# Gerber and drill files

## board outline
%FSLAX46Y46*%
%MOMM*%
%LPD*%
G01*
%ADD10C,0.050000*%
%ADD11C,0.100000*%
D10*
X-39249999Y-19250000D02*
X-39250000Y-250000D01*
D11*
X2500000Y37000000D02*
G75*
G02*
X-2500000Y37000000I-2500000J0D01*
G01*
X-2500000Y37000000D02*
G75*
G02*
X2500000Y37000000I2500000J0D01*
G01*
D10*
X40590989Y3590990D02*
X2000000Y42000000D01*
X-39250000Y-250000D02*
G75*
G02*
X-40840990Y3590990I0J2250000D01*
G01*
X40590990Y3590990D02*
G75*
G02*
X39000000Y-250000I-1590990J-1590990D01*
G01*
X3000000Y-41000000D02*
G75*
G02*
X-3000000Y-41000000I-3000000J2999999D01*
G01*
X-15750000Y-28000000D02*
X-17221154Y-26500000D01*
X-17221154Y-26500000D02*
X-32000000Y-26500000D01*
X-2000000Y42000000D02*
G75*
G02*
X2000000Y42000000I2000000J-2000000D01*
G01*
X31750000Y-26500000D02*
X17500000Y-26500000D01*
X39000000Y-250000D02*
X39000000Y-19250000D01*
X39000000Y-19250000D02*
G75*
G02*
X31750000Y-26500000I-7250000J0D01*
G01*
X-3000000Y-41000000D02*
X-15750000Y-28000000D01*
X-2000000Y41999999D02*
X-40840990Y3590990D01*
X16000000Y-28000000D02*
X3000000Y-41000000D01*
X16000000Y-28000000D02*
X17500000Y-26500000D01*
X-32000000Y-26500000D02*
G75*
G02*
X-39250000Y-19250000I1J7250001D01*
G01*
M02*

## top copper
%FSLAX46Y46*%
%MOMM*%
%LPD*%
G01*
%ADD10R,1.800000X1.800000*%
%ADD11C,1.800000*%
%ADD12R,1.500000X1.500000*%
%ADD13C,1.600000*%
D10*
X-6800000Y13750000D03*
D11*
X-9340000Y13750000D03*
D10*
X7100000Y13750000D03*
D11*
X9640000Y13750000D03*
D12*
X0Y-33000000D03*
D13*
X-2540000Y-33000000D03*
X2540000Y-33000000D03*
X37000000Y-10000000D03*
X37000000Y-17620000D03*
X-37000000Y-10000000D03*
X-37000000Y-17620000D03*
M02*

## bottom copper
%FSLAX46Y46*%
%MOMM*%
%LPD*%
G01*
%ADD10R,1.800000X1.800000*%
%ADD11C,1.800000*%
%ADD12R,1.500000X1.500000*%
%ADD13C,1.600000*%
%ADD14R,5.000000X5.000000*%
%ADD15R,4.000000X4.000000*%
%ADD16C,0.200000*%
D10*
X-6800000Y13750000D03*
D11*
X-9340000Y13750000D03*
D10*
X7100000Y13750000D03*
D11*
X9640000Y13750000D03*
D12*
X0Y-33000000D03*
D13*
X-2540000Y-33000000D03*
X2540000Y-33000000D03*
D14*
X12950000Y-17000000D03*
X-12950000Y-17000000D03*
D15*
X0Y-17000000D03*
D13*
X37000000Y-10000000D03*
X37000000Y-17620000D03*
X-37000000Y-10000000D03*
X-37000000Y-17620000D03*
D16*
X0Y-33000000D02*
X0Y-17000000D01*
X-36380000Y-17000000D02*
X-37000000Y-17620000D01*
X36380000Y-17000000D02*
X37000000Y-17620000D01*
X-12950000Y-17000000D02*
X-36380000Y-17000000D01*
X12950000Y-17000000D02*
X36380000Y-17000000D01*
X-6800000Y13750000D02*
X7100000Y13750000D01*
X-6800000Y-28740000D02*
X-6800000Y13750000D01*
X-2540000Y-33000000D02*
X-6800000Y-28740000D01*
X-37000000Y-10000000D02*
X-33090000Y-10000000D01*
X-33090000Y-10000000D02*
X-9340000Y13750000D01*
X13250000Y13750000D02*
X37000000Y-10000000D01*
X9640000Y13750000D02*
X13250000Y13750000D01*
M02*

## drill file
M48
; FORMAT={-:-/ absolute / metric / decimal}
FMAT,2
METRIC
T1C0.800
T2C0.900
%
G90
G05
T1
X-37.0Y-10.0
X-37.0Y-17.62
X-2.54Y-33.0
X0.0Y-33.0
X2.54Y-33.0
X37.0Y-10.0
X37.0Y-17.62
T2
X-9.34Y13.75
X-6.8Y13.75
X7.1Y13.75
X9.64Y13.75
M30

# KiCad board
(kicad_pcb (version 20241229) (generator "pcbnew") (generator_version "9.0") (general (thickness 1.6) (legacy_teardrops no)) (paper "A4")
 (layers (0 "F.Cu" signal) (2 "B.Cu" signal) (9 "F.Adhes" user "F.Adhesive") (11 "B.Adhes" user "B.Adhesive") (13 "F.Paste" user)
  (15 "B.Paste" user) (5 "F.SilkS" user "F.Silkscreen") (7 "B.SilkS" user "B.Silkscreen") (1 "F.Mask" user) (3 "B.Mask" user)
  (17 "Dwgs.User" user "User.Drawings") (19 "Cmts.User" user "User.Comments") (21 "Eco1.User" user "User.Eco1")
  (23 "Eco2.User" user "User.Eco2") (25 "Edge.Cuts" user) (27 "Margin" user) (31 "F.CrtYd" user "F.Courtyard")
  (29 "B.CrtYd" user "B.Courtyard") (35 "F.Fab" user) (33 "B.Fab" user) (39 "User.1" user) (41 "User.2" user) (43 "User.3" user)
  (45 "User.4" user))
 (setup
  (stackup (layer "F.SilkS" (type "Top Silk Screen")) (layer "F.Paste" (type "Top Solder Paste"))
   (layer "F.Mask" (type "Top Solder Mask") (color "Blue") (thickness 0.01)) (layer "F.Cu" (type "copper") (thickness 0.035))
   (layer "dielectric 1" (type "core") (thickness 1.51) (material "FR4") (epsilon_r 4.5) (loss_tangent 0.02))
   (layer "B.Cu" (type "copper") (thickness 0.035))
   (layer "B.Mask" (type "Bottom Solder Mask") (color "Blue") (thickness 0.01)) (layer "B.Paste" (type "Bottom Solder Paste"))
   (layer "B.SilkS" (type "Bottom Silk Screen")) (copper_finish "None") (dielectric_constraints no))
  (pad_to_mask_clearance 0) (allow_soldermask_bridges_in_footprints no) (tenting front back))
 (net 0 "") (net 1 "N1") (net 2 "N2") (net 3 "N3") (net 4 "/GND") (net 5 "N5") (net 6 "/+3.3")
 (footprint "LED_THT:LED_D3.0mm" (layer "F.Cu") (at -6.8 -13.75 180)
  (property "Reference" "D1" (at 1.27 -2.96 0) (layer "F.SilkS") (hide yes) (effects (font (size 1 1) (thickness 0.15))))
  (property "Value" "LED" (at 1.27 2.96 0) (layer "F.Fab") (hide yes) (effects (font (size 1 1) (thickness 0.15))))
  (pad "1" thru_hole rect (at 0 0 180) (size 1.8 1.8) (drill 0.9) (layers "*.Cu" "*.Mask") (remove_unused_layers no) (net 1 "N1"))
  (pad "2" thru_hole circle (at 2.54 0 180) (size 1.8 1.8) (drill 0.9) (layers "*.Cu" "*.Mask") (remove_unused_layers no) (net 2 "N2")))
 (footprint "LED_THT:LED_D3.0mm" (layer "F.Cu") (at 7.1 -13.75)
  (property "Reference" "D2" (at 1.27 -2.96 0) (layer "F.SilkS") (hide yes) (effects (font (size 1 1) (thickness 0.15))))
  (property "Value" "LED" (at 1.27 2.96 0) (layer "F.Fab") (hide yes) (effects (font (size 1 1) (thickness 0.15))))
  (pad "1" thru_hole rect (at 0 0) (size 1.8 1.8) (drill 0.9) (layers "*.Cu" "*.Mask") (remove_unused_layers no) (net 1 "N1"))
  (pad "2" thru_hole circle (at 2.54 0) (size 1.8 1.8) (drill 0.9) (layers "*.Cu" "*.Mask") (remove_unused_layers no) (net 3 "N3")))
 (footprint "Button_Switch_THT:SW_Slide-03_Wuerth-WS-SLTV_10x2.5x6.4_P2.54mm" (layer "B.Cu") (at 0 33)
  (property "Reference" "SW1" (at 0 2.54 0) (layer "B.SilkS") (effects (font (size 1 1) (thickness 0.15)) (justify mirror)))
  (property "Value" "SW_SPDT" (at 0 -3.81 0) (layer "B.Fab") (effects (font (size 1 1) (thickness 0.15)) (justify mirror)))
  (pad "1" thru_hole rect (at 0 0) (size 1.5 1.5) (drill 0.8) (layers "*.Cu" "*.Mask") (remove_unused_layers no) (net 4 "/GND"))
  (pad "2" thru_hole circle (at -2.54 0) (size 1.6 1.6) (drill 0.8) (layers "*.Cu" "*.Mask") (remove_unused_layers no) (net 1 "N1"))
  (pad "3" thru_hole circle (at 2.54 0) (size 1.6 1.6) (drill 0.8) (layers "*.Cu" "*.Mask") (remove_unused_layers no) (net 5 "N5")))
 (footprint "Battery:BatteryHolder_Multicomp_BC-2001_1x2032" (layer "B.Cu") (at 0 17 180)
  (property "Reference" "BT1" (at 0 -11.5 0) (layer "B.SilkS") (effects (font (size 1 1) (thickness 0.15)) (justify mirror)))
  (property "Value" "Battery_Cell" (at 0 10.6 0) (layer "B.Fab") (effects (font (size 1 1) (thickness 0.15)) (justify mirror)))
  (pad "1" smd rect (at -12.95 0 180) (size 5 5) (layers "B.Cu" "B.Mask" "B.Paste") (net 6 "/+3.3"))
  (pad "1" smd rect (at 12.95 0 180) (size 5 5) (layers "B.Cu" "B.Mask" "B.Paste") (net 6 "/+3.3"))
  (pad "2" smd rect (at 0 0 180) (size 4 4) (layers "B.Cu" "B.Mask" "B.Paste") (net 4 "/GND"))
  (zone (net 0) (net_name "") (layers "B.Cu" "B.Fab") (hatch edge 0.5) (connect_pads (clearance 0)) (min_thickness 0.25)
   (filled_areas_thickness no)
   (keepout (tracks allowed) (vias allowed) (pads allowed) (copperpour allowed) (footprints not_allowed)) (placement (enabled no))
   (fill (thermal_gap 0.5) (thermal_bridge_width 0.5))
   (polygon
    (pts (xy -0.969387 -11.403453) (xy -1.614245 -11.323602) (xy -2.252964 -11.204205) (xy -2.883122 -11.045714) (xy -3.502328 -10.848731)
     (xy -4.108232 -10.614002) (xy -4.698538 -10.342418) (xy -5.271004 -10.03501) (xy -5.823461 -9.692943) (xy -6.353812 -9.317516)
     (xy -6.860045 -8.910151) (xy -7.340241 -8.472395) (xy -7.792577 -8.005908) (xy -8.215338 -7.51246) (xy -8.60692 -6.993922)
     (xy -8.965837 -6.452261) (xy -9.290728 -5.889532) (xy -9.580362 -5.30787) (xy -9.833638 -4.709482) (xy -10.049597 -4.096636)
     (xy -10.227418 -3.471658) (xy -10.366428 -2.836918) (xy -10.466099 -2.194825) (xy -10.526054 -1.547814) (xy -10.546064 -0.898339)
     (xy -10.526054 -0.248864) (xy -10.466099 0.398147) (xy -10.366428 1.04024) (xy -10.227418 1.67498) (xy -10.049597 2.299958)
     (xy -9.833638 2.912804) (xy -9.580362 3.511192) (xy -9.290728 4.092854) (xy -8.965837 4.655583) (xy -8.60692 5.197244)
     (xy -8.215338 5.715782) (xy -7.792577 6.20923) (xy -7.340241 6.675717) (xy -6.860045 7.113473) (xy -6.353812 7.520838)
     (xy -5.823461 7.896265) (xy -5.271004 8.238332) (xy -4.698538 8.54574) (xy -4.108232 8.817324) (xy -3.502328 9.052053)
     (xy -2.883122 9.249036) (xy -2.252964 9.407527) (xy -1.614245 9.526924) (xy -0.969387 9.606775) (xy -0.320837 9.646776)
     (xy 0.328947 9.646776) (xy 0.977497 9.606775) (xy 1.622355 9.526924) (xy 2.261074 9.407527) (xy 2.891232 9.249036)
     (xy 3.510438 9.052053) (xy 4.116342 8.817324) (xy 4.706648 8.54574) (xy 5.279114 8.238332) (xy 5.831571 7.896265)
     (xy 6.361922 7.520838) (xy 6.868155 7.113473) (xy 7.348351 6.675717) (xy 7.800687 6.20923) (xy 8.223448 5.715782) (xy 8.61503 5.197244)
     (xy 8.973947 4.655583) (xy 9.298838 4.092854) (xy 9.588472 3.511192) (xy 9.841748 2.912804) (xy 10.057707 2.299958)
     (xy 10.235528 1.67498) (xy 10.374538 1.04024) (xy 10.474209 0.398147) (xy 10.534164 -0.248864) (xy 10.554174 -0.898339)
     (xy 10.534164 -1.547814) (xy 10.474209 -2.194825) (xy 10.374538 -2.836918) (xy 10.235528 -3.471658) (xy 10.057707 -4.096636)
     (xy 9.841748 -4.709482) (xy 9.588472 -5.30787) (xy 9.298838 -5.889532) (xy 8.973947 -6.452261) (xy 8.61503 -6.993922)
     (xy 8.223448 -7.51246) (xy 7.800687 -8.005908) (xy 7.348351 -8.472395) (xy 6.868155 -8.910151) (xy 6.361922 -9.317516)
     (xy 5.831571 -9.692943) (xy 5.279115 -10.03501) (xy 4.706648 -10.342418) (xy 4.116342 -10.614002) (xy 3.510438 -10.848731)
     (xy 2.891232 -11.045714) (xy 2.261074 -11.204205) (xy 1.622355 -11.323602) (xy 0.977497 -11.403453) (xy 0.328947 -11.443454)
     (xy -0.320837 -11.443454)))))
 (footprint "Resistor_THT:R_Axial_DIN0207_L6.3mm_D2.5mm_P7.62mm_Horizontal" (layer "B.Cu") (at 37 10 -90)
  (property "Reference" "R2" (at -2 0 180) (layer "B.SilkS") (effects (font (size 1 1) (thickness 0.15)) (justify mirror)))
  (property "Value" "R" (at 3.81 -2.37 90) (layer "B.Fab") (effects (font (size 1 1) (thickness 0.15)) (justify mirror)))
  (pad "1" thru_hole circle (at 0 0 270) (size 1.6 1.6) (drill 0.8) (layers "*.Cu" "*.Mask") (remove_unused_layers no) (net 3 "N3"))
  (pad "2" thru_hole circle (at 7.62 0 270) (size 1.6 1.6) (drill 0.8) (layers "*.Cu" "*.Mask") (remove_unused_layers no) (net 6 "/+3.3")))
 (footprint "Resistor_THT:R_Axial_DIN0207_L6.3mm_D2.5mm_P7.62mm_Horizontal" (layer "B.Cu") (at -37 10 -90)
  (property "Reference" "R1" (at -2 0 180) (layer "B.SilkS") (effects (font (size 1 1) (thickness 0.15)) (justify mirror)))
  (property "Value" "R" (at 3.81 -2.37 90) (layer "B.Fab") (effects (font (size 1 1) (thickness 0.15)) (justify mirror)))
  (pad "1" thru_hole circle (at 0 0 270) (size 1.6 1.6) (drill 0.8) (layers "*.Cu" "*.Mask") (remove_unused_layers no) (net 2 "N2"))
  (pad "2" thru_hole circle (at 7.62 0 270) (size 1.6 1.6) (drill 0.8) (layers "*.Cu" "*.Mask") (remove_unused_layers no) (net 6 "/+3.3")))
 (gr_line (start -39.249999 19.25) (end -39.25 0.25) (stroke (width 0.05) (type default)) (layer "Edge.Cuts"))
 (gr_circle (center 0 -37) (end 2.5 -37) (stroke (width 0.1) (type solid)) (fill no) (layer "Edge.Cuts"))
 (gr_line (start 40.590989 -3.59099) (end 2 -42) (stroke (width 0.05) (type default)) (layer "Edge.Cuts"))
 (gr_arc (start -39.25 0.25) (mid -41.328729 -1.138962) (end -40.84099 -3.59099) (stroke (width 0.05) (type default)) (layer "Edge.Cuts"))
 (gr_arc (start 40.59099 -3.59099) (mid 41.078729 -1.138962) (end 39 0.25) (stroke (width 0.05) (type default)) (layer "Edge.Cuts"))
 (gr_arc (start 3 41) (mid 0 42.242641) (end -3 41) (stroke (width 0.05) (type default)) (layer "Edge.Cuts"))
 (gr_line (start -15.75 28) (end -17.221154 26.5) (stroke (width 0.05) (type default)) (layer "Edge.Cuts"))
 (gr_line (start -17.221154 26.5) (end -32 26.5) (stroke (width 0.05) (type default)) (layer "Edge.Cuts"))
 (gr_arc (start -2 -42) (mid 0 -42.828427) (end 2 -42) (stroke (width 0.05) (type default)) (layer "Edge.Cuts"))
 (gr_line (start 31.75 26.5) (end 17.5 26.5) (stroke (width 0.05) (type default)) (layer "Edge.Cuts"))
 (gr_line (start 39 0.25) (end 39 19.25) (stroke (width 0.05) (type default)) (layer "Edge.Cuts"))
 (gr_arc (start 39 19.25) (mid 36.876524 24.376524) (end 31.75 26.5) (stroke (width 0.05) (type default)) (layer "Edge.Cuts"))
 (gr_line (start -3 41) (end -15.75 28) (stroke (width 0.05) (type default)) (layer "Edge.Cuts"))
 (gr_line (start -2 -41.999999) (end -40.84099 -3.59099) (stroke (width 0.05) (type default)) (layer "Edge.Cuts"))
 (gr_line (start 16 28) (end 3 41) (stroke (width 0.05) (type default)) (layer "Edge.Cuts"))
 (gr_line (start 16 28) (end 17.5 26.5) (stroke (width 0.05) (type default)) (layer "Edge.Cuts"))
 (gr_arc (start -32 26.5) (mid -37.126524 24.376524) (end -39.25 19.25) (stroke (width 0.05) (type default)) (layer "Edge.Cuts"))
 (segment (start 0 33) (end 0 17) (width 0.2) (layer "B.Cu") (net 4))
 (segment (start -36.38 17) (end -37 17.62) (width 0.2) (layer "B.Cu") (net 6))
 (segment (start 36.38 17) (end 37 17.62) (width 0.2) (layer "B.Cu") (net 6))
 (segment (start -12.95 17) (end -36.38 17) (width 0.2) (layer "B.Cu") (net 6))
 (segment (start 12.95 17) (end 36.38 17) (width 0.2) (layer "B.Cu") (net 6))
 (segment (start -6.8 -13.75) (end 7.1 -13.75) (width 0.2) (layer "B.Cu") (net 1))
 (segment (start -6.8 28.74) (end -6.8 -13.75) (width 0.2) (layer "B.Cu") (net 1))
 (segment (start -2.54 33) (end -6.8 28.74) (width 0.2) (layer "B.Cu") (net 1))
 (segment (start -37 10) (end -33.09 10) (width 0.2) (layer "B.Cu") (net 2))
 (segment (start -33.09 10) (end -9.34 -13.75) (width 0.2) (layer "B.Cu") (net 2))
 (segment (start 13.25 -13.75) (end 37 10) (width 0.2) (layer "B.Cu") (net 3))
 (segment (start 9.64 -13.75) (end 13.25 -13.75) (width 0.2) (layer "B.Cu") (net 3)))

